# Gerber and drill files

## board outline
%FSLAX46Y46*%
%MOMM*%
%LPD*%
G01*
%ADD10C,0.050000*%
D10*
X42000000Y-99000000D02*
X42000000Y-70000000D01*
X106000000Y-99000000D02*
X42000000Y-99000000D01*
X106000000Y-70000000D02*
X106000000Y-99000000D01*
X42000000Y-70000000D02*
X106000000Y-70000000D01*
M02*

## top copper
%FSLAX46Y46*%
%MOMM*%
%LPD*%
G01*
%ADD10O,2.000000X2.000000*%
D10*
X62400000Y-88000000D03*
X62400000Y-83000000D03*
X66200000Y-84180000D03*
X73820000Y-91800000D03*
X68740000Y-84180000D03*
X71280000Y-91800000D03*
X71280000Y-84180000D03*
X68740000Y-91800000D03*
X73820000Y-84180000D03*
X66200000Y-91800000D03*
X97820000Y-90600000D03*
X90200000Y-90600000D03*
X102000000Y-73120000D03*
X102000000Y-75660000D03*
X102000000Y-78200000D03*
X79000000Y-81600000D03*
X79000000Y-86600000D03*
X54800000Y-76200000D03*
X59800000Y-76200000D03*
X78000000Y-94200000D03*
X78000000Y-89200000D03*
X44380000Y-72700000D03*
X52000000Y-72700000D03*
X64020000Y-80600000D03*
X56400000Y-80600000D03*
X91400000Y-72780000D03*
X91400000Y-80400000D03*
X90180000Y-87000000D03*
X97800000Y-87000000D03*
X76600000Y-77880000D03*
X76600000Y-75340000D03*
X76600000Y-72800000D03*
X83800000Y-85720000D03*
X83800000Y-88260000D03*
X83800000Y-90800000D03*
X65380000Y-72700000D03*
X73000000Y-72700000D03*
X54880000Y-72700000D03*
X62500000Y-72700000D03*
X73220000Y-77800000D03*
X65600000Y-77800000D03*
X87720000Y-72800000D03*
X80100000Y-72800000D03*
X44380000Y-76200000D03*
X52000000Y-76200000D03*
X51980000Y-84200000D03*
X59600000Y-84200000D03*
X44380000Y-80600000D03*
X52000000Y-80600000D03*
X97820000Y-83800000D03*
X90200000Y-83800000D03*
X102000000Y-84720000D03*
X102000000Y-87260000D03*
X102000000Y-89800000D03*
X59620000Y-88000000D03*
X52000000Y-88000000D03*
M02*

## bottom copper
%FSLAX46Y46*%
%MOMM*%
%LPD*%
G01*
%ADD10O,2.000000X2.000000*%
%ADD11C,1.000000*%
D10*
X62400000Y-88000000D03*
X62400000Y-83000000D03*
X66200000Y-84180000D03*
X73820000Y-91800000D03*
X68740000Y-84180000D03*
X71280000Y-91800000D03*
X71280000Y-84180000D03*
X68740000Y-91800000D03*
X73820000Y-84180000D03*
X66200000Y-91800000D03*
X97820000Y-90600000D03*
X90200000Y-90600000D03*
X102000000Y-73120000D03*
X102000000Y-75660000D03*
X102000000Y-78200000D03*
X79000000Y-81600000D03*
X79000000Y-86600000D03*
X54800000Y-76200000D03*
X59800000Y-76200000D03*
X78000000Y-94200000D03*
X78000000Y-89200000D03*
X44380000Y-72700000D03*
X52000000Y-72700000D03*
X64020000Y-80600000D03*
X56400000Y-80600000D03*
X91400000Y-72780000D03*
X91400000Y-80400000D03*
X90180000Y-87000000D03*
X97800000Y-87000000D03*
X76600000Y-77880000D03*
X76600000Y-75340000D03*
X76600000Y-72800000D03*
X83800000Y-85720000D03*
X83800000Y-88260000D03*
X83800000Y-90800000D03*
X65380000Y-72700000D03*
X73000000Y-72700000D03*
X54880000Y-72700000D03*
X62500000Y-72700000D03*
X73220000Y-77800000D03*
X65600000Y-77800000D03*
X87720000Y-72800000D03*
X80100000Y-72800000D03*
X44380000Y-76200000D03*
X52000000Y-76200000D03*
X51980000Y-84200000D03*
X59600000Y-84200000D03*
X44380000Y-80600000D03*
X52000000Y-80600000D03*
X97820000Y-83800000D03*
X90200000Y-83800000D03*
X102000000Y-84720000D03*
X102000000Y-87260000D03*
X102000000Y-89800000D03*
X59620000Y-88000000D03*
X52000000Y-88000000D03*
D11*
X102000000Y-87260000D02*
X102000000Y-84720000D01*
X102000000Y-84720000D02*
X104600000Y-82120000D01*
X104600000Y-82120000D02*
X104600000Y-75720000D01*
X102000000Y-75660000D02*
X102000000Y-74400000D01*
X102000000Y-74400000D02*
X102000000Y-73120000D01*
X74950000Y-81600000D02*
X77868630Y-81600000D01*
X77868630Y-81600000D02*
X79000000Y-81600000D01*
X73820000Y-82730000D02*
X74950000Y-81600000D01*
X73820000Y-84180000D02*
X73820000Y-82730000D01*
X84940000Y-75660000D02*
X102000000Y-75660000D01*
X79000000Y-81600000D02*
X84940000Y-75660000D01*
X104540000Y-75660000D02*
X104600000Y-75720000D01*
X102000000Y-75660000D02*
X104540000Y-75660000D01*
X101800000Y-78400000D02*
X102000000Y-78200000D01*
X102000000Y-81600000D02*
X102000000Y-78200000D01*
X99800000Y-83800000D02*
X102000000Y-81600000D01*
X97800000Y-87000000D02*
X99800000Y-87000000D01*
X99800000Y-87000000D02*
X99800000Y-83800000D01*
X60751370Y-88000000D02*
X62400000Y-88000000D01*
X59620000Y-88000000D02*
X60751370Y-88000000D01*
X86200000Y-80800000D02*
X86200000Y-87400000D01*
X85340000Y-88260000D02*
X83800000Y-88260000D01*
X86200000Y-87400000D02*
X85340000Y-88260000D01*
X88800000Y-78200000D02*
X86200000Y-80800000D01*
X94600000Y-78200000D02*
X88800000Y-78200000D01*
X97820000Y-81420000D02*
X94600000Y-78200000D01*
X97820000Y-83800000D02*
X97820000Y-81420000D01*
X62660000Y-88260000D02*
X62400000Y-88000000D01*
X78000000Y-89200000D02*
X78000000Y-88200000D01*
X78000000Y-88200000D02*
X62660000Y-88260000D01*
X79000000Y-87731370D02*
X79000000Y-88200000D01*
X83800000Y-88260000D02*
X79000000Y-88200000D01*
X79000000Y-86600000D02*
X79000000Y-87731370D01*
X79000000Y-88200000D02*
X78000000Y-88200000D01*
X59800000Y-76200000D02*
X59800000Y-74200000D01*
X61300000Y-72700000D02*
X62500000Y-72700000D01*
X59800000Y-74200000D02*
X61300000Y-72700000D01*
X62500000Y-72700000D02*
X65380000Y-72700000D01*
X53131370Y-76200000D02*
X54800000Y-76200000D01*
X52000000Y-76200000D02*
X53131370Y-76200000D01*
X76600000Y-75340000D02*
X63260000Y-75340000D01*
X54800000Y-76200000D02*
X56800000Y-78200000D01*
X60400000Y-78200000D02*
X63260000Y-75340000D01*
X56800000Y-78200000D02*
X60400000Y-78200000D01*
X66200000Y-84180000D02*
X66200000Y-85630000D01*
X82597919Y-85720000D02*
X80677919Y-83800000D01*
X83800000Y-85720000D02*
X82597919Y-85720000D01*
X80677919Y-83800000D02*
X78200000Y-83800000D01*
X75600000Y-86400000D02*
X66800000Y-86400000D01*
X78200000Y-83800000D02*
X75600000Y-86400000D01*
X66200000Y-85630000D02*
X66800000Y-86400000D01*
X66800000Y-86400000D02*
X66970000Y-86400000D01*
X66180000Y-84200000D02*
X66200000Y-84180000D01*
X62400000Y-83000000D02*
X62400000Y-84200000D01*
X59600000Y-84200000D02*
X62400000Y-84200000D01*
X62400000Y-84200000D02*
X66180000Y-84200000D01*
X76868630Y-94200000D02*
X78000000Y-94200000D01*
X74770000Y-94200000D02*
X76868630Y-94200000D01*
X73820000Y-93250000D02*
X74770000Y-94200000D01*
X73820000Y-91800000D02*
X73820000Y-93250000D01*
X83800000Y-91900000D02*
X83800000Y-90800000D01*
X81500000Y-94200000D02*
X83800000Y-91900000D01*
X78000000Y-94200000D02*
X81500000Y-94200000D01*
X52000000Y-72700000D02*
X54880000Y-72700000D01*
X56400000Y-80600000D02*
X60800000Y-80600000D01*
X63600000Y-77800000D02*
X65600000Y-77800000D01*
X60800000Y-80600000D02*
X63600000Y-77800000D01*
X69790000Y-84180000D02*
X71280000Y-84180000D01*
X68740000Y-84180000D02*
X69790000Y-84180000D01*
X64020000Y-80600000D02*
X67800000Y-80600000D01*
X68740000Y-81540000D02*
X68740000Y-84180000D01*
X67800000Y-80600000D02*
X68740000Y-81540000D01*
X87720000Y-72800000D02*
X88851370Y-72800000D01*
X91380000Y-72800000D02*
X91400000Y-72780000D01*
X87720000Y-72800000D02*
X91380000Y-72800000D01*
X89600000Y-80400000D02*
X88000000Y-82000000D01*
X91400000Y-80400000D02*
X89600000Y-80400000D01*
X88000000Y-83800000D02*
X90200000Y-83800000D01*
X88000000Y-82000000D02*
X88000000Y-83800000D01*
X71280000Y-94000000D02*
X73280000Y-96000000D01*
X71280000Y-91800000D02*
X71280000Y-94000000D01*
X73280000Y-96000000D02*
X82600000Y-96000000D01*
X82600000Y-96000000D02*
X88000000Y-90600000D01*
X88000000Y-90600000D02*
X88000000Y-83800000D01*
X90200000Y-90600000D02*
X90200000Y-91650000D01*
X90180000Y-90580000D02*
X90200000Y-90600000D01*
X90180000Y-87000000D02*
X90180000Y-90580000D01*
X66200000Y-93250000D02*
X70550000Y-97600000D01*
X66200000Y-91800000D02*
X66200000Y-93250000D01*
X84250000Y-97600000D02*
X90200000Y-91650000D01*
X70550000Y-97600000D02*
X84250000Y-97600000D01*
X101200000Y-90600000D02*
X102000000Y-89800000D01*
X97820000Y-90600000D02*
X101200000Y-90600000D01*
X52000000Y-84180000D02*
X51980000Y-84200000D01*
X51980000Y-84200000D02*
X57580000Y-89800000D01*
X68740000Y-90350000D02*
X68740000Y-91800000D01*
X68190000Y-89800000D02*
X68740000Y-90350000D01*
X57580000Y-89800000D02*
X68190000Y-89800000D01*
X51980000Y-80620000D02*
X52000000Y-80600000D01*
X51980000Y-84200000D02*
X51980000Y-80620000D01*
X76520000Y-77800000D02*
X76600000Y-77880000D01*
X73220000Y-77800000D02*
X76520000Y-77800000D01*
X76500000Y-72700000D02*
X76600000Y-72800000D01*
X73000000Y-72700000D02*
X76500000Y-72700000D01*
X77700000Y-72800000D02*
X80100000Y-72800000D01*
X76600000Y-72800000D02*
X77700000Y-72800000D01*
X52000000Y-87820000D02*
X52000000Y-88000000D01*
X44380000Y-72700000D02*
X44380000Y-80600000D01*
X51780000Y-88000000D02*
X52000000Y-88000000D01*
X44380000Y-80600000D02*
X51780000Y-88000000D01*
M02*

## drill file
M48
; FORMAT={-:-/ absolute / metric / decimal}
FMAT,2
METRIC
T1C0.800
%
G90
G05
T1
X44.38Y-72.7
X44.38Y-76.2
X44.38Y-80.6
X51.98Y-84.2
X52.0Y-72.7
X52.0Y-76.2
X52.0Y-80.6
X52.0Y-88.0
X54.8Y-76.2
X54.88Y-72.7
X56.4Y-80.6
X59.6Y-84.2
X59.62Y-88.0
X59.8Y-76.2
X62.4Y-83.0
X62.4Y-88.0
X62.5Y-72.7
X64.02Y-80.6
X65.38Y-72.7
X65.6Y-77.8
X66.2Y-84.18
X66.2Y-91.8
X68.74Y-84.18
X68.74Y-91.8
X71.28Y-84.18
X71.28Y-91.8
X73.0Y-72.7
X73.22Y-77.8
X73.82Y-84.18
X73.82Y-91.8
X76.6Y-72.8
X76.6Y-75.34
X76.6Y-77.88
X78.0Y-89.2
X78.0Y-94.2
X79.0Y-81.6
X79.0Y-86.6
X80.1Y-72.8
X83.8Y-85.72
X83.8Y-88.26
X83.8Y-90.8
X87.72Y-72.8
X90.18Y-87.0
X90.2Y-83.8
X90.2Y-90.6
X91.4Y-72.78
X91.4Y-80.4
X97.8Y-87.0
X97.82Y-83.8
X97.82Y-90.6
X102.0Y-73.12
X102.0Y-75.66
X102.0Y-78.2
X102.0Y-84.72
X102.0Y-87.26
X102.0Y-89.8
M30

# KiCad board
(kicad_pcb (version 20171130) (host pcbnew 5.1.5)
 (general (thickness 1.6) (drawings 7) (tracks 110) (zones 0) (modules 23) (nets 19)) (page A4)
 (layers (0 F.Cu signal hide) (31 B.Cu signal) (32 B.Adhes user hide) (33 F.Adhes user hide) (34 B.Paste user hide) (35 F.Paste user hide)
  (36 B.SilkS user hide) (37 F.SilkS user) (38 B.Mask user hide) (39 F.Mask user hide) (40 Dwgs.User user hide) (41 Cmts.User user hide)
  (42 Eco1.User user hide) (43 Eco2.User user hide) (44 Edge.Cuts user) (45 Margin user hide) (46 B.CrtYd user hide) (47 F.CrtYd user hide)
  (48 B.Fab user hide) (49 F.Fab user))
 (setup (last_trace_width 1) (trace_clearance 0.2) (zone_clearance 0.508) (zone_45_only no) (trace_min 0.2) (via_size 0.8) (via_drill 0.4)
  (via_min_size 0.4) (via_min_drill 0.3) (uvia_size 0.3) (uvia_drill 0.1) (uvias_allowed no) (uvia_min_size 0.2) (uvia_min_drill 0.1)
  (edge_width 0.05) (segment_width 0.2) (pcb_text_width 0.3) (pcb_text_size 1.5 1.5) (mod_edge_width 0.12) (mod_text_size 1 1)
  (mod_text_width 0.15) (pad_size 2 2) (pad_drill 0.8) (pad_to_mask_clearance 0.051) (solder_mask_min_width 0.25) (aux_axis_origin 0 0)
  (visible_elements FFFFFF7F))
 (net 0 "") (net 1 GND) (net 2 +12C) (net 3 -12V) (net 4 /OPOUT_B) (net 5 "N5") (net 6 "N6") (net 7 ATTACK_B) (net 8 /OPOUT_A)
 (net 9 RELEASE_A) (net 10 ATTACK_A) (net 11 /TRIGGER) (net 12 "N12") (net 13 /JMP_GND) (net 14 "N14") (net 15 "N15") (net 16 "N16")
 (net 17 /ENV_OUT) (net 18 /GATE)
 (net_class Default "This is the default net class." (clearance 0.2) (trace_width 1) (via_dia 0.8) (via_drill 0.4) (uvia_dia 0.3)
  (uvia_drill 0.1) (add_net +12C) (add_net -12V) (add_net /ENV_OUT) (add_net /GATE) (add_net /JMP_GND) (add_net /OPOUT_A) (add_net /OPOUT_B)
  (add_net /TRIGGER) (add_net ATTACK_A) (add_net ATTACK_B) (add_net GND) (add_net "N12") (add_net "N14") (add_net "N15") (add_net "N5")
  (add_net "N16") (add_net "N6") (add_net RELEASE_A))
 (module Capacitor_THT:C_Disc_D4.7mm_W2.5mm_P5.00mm (layer F.Cu) (at 62.4 83 270)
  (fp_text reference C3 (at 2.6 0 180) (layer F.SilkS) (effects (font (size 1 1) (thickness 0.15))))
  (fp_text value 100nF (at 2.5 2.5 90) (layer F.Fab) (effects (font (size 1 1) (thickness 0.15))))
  (pad 2 thru_hole oval (at 5 0 270) (size 2 2) (drill 0.8) (layers *.Cu *.Mask) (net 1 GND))
  (pad 1 thru_hole oval (at 0 0 270) (size 2 2) (drill 0.8) (layers *.Cu *.Mask) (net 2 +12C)))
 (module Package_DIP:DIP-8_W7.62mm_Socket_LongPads (layer F.Cu) (at 66.2 91.8 90)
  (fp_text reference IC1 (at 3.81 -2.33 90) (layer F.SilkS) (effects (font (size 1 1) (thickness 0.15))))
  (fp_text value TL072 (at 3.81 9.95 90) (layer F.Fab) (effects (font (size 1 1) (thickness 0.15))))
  (pad 8 thru_hole oval (at 7.62 0 90) (size 2 2) (drill 0.8) (layers *.Cu *.Mask) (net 2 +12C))
  (pad 4 thru_hole oval (at 0 7.62 90) (size 2 2) (drill 0.8) (layers *.Cu *.Mask) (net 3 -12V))
  (pad 7 thru_hole oval (at 7.62 2.54 90) (size 2 2) (drill 0.8) (layers *.Cu *.Mask) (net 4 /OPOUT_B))
  (pad 3 thru_hole oval (at 0 5.08 90) (size 2 2) (drill 0.8) (layers *.Cu *.Mask) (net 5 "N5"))
  (pad 6 thru_hole oval (at 7.62 5.08 90) (size 2 2) (drill 0.8) (layers *.Cu *.Mask) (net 4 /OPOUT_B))
  (pad 2 thru_hole oval (at 0 2.54 90) (size 2 2) (drill 0.8) (layers *.Cu *.Mask) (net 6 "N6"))
  (pad 5 thru_hole oval (at 7.62 7.62 90) (size 2 2) (drill 0.8) (layers *.Cu *.Mask) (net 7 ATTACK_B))
  (pad 1 thru_hole oval (at 0 0 90) (size 2 2) (drill 0.8) (layers *.Cu *.Mask) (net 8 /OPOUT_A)))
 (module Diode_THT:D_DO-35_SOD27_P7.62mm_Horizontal (layer F.Cu) (at 90.2 90.6)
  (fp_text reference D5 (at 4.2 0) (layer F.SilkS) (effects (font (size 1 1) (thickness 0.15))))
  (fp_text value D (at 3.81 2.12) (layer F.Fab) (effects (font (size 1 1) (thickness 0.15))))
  (pad 2 thru_hole oval (at 7.62 0) (size 2 2) (drill 0.8) (layers *.Cu *.Mask) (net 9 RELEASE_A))
  (pad 1 thru_hole oval (at 0 0) (size 2 2) (drill 0.8) (layers *.Cu *.Mask) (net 8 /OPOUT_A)))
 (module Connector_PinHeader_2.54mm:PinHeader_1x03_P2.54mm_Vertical (layer F.Cu) (at 102 78.2 180)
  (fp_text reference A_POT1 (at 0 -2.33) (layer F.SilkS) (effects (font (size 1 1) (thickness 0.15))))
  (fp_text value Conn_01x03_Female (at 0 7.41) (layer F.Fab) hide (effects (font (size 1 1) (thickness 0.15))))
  (pad 3 thru_hole oval (at 0 5.08 180) (size 2 2) (drill 0.8) (layers *.Cu *.Mask) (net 7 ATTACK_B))
  (pad 2 thru_hole oval (at 0 2.54 180) (size 2 2) (drill 0.8) (layers *.Cu *.Mask) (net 7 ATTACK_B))
  (pad 1 thru_hole oval (at 0 0 180) (size 2 2) (drill 0.8) (layers *.Cu *.Mask) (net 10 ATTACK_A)))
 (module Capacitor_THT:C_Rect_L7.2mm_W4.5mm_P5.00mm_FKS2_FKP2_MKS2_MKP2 (layer F.Cu) (at 79 86.6 90)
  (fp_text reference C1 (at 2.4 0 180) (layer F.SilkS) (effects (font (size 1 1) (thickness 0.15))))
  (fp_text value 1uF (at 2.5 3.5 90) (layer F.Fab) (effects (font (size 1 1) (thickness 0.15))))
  (pad 2 thru_hole oval (at 5 0 90) (size 2 2) (drill 0.8) (layers *.Cu *.Mask) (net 7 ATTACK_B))
  (pad 1 thru_hole oval (at 0 0 90) (size 2 2) (drill 0.8) (layers *.Cu *.Mask) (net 1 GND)))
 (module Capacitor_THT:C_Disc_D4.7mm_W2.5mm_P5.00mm (layer F.Cu) (at 59.8 76.2 180)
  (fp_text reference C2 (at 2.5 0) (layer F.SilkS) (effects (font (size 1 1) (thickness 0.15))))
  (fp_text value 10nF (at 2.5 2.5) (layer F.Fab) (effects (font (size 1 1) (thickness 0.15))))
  (pad 2 thru_hole oval (at 5 0 180) (size 2 2) (drill 0.8) (layers *.Cu *.Mask) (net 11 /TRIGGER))
  (pad 1 thru_hole oval (at 0 0 180) (size 2 2) (drill 0.8) (layers *.Cu *.Mask) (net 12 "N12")))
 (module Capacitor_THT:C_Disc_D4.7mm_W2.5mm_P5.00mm (layer F.Cu) (at 78 89.2 270)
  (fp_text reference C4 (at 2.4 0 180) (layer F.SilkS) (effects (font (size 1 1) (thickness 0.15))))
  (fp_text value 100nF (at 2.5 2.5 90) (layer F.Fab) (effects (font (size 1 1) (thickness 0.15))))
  (pad 2 thru_hole oval (at 5 0 270) (size 2 2) (drill 0.8) (layers *.Cu *.Mask) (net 3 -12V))
  (pad 1 thru_hole oval (at 0 0 270) (size 2 2) (drill 0.8) (layers *.Cu *.Mask) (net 1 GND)))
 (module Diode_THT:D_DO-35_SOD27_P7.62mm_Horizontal (layer F.Cu) (at 52 72.7 180)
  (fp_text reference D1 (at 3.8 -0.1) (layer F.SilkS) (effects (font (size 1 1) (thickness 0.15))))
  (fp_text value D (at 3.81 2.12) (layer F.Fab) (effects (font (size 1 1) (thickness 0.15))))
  (pad 2 thru_hole oval (at 7.62 0 180) (size 2 2) (drill 0.8) (layers *.Cu *.Mask) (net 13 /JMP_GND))
  (pad 1 thru_hole oval (at 0 0 180) (size 2 2) (drill 0.8) (layers *.Cu *.Mask) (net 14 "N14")))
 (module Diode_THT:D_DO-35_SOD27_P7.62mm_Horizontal (layer F.Cu) (at 56.4 80.6)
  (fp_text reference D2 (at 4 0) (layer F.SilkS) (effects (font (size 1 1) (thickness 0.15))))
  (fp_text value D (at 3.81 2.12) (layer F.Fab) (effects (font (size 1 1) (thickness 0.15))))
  (pad 2 thru_hole oval (at 7.62 0) (size 2 2) (drill 0.8) (layers *.Cu *.Mask) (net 4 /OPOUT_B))
  (pad 1 thru_hole oval (at 0 0) (size 2 2) (drill 0.8) (layers *.Cu *.Mask) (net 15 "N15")))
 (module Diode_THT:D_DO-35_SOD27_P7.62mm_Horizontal (layer F.Cu) (at 91.4 80.4 90)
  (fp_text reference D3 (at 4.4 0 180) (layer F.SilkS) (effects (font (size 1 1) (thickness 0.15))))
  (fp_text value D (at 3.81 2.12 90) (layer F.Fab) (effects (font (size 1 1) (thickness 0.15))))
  (pad 2 thru_hole oval (at 7.62 0 90) (size 2 2) (drill 0.8) (layers *.Cu *.Mask) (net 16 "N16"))
  (pad 1 thru_hole oval (at 0 0 90) (size 2 2) (drill 0.8) (layers *.Cu *.Mask) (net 5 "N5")))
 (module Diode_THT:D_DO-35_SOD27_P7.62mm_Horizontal (layer F.Cu) (at 97.8 87 180)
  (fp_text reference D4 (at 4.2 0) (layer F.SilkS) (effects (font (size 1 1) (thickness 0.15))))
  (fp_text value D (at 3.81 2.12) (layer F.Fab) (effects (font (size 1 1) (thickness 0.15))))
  (pad 2 thru_hole oval (at 7.62 0 180) (size 2 2) (drill 0.8) (layers *.Cu *.Mask) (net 8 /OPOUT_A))
  (pad 1 thru_hole oval (at 0 0 180) (size 2 2) (drill 0.8) (layers *.Cu *.Mask) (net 10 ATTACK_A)))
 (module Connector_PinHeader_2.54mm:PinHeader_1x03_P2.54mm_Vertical (layer F.Cu) (at 76.6 72.8)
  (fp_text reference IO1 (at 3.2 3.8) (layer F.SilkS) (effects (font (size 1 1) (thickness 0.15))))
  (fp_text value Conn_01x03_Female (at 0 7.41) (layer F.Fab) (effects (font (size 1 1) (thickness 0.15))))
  (pad 3 thru_hole oval (at 0 5.08) (size 2 2) (drill 0.8) (layers *.Cu *.Mask) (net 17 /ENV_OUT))
  (pad 2 thru_hole oval (at 0 2.54) (size 2 2) (drill 0.8) (layers *.Cu *.Mask) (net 11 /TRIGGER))
  (pad 1 thru_hole oval (at 0 0) (size 2 2) (drill 0.8) (layers *.Cu *.Mask) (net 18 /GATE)))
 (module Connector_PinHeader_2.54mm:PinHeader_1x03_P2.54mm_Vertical (layer F.Cu) (at 83.8 90.8 180)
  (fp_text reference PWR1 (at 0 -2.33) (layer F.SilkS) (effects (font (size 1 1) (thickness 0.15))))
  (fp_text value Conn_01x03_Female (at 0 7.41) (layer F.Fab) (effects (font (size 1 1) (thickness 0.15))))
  (pad 3 thru_hole oval (at 0 5.08 180) (size 2 2) (drill 0.8) (layers *.Cu *.Mask) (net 2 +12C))
  (pad 2 thru_hole oval (at 0 2.54 180) (size 2 2) (drill 0.8) (layers *.Cu *.Mask) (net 1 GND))
  (pad 1 thru_hole oval (at 0 0 180) (size 2 2) (drill 0.8) (layers *.Cu *.Mask) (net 3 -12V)))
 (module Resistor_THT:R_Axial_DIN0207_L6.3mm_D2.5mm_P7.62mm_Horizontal (layer F.Cu) (at 73 72.7 180)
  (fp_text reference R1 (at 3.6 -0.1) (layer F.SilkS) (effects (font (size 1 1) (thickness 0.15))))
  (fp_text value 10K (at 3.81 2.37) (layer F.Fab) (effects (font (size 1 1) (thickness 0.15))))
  (pad 2 thru_hole oval (at 7.62 0 180) (size 2 2) (drill 0.8) (layers *.Cu *.Mask) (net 12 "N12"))
  (pad 1 thru_hole oval (at 0 0 180) (size 2 2) (drill 0.8) (layers *.Cu *.Mask) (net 18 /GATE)))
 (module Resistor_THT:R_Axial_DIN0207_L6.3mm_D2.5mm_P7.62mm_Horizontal (layer F.Cu) (at 62.5 72.7 180)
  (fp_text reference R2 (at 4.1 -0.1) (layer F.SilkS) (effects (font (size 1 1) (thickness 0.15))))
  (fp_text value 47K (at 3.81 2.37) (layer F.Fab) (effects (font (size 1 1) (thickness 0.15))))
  (pad 2 thru_hole oval (at 7.62 0 180) (size 2 2) (drill 0.8) (layers *.Cu *.Mask) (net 14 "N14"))
  (pad 1 thru_hole oval (at 0 0 180) (size 2 2) (drill 0.8) (layers *.Cu *.Mask) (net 12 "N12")))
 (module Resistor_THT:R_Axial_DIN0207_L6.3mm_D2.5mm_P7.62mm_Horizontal (layer F.Cu) (at 65.6 77.8)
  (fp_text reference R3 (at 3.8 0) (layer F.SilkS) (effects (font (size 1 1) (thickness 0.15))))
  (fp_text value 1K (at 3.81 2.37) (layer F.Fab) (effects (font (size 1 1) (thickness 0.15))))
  (pad 2 thru_hole oval (at 7.62 0) (size 2 2) (drill 0.8) (layers *.Cu *.Mask) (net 17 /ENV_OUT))
  (pad 1 thru_hole oval (at 0 0) (size 2 2) (drill 0.8) (layers *.Cu *.Mask) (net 15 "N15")))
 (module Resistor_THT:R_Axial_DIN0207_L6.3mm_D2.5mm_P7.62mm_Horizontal (layer F.Cu) (at 80.1 72.8)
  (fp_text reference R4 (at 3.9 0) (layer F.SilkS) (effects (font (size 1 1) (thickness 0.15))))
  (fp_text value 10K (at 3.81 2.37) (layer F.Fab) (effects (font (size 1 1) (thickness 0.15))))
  (pad 2 thru_hole oval (at 7.62 0) (size 2 2) (drill 0.8) (layers *.Cu *.Mask) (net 16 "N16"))
  (pad 1 thru_hole oval (at 0 0) (size 2 2) (drill 0.8) (layers *.Cu *.Mask) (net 18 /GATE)))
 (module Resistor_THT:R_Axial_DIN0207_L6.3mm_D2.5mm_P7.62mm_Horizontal (layer F.Cu) (at 52 76.2 180)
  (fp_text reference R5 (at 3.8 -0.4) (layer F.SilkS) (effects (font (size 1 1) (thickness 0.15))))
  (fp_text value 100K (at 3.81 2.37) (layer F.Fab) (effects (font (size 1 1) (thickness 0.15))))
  (pad 2 thru_hole oval (at 7.62 0 180) (size 2 2) (drill 0.8) (layers *.Cu *.Mask) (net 13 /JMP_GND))
  (pad 1 thru_hole oval (at 0 0 180) (size 2 2) (drill 0.8) (layers *.Cu *.Mask) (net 11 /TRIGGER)))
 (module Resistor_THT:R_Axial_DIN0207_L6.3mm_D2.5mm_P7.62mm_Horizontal (layer F.Cu) (at 59.6 84.2 180)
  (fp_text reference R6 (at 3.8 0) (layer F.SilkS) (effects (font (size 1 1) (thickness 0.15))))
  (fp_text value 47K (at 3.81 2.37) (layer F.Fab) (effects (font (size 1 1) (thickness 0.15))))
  (pad 2 thru_hole oval (at 7.62 0 180) (size 2 2) (drill 0.8) (layers *.Cu *.Mask) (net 6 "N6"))
  (pad 1 thru_hole oval (at 0 0 180) (size 2 2) (drill 0.8) (layers *.Cu *.Mask) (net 2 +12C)))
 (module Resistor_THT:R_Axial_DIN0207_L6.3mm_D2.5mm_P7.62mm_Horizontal (layer F.Cu) (at 52 80.6 180)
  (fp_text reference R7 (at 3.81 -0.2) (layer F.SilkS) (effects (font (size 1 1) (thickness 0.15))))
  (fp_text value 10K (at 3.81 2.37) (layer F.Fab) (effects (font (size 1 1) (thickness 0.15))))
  (pad 2 thru_hole oval (at 7.62 0 180) (size 2 2) (drill 0.8) (layers *.Cu *.Mask) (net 13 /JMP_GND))
  (pad 1 thru_hole oval (at 0 0 180) (size 2 2) (drill 0.8) (layers *.Cu *.Mask) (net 6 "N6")))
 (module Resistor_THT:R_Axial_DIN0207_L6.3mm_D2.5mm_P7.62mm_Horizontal (layer F.Cu) (at 90.2 83.8)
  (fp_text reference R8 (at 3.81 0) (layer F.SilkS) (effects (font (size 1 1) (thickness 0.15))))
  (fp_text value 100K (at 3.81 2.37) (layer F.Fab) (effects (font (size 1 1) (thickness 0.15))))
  (pad 2 thru_hole oval (at 7.62 0) (size 2 2) (drill 0.8) (layers *.Cu *.Mask) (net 1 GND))
  (pad 1 thru_hole oval (at 0 0) (size 2 2) (drill 0.8) (layers *.Cu *.Mask) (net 5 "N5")))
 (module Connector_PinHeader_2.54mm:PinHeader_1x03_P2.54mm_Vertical (layer F.Cu) (at 102 89.8 180)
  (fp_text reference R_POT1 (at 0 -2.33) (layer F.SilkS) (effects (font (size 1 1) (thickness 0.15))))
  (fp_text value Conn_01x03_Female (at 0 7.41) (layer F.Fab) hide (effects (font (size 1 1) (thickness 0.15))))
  (pad 3 thru_hole oval (at 0 5.08 180) (size 2 2) (drill 0.8) (layers *.Cu *.Mask) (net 7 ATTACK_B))
  (pad 2 thru_hole oval (at 0 2.54 180) (size 2 2) (drill 0.8) (layers *.Cu *.Mask) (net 7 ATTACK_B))
  (pad 1 thru_hole oval (at 0 0 180) (size 2 2) (drill 0.8) (layers *.Cu *.Mask) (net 9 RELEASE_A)))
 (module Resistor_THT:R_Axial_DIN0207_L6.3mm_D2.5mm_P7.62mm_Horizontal (layer F.Cu) (at 52 88)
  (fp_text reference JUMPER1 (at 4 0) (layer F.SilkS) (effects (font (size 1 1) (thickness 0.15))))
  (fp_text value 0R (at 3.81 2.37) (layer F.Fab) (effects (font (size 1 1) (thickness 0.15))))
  (pad 2 thru_hole oval (at 7.62 0) (size 2 2) (drill 0.8) (layers *.Cu *.Mask) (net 1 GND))
  (pad 1 thru_hole oval (at 0 0) (size 2 2) (drill 0.8) (layers *.Cu *.Mask) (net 13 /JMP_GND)))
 (gr_line (start 42 99) (end 42 70) (layer Edge.Cuts) (width 0.05))
 (gr_line (start 106 99) (end 42 99) (layer Edge.Cuts) (width 0.05))
 (gr_line (start 106 70) (end 106 99) (layer Edge.Cuts) (width 0.05))
 (gr_line (start 42 70) (end 106 70) (layer Edge.Cuts) (width 0.05))
 (segment (start 102 87.26) (end 102 84.72) (width 1) (layer B.Cu) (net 7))
 (segment (start 102 84.72) (end 104.6 82.12) (width 1) (layer B.Cu) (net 7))
 (segment (start 104.6 82.12) (end 104.6 75.72) (width 1) (layer B.Cu) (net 7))
 (segment (start 102 75.66) (end 102 74.4) (width 1) (layer B.Cu) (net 7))
 (segment (start 102 74.4) (end 102 73.12) (width 1) (layer B.Cu) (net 7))
 (segment (start 74.95 81.6) (end 77.86863 81.6) (width 1) (layer B.Cu) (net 7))
 (segment (start 77.86863 81.6) (end 79 81.6) (width 1) (layer B.Cu) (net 7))
 (segment (start 73.82 82.73) (end 74.95 81.6) (width 1) (layer B.Cu) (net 7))
 (segment (start 73.82 84.18) (end 73.82 82.73) (width 1) (layer B.Cu) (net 7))
 (segment (start 84.94 75.66) (end 102 75.66) (width 1) (layer B.Cu) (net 7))
 (segment (start 79 81.6) (end 84.94 75.66) (width 1) (layer B.Cu) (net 7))
 (segment (start 104.54 75.66) (end 104.6 75.72) (width 1) (layer B.Cu) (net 7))
 (segment (start 102 75.66) (end 104.54 75.66) (width 1) (layer B.Cu) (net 7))
 (segment (start 101.8 78.4) (end 102 78.2) (width 1) (layer B.Cu) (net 10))
 (segment (start 102 81.6) (end 102 78.2) (width 1) (layer B.Cu) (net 10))
 (segment (start 99.8 83.8) (end 102 81.6) (width 1) (layer B.Cu) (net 10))
 (segment (start 97.8 87) (end 99.8 87) (width 1) (layer B.Cu) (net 10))
 (segment (start 99.8 87) (end 99.8 83.8) (width 1) (layer B.Cu) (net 10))
 (segment (start 60.75137 88) (end 62.4 88) (width 1) (layer B.Cu) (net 1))
 (segment (start 59.62 88) (end 60.75137 88) (width 1) (layer B.Cu) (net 1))
 (segment (start 86.2 80.8) (end 86.2 87.4) (width 1) (layer B.Cu) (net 1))
 (segment (start 85.34 88.26) (end 83.8 88.26) (width 1) (layer B.Cu) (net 1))
 (segment (start 86.2 87.4) (end 85.34 88.26) (width 1) (layer B.Cu) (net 1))
 (segment (start 88.8 78.2) (end 86.2 80.8) (width 1) (layer B.Cu) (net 1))
 (segment (start 94.6 78.2) (end 88.8 78.2) (width 1) (layer B.Cu) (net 1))
 (segment (start 97.82 81.42) (end 94.6 78.2) (width 1) (layer B.Cu) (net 1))
 (segment (start 97.82 83.8) (end 97.82 81.42) (width 1) (layer B.Cu) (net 1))
 (segment (start 62.66 88.26) (end 62.4 88) (width 1) (layer B.Cu) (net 1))
 (segment (start 78 89.2) (end 78 88.2) (width 1) (layer B.Cu) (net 1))
 (segment (start 78 88.2) (end 62.66 88.26) (width 1) (layer B.Cu) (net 1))
 (segment (start 79 87.73137) (end 79 88.2) (width 1) (layer B.Cu) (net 1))
 (segment (start 83.8 88.26) (end 79 88.2) (width 1) (layer B.Cu) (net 1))
 (segment (start 79 86.6) (end 79 87.73137) (width 1) (layer B.Cu) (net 1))
 (segment (start 79 88.2) (end 78 88.2) (width 1) (layer B.Cu) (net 1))
 (segment (start 59.8 76.2) (end 59.8 74.2) (width 1) (layer B.Cu) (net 12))
 (segment (start 61.3 72.7) (end 62.5 72.7) (width 1) (layer B.Cu) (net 12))
 (segment (start 59.8 74.2) (end 61.3 72.7) (width 1) (layer B.Cu) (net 12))
 (segment (start 62.5 72.7) (end 65.38 72.7) (width 1) (layer B.Cu) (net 12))
 (segment (start 53.13137 76.2) (end 54.8 76.2) (width 1) (layer B.Cu) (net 11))
 (segment (start 52 76.2) (end 53.13137 76.2) (width 1) (layer B.Cu) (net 11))
 (segment (start 76.6 75.34) (end 63.26 75.34) (width 1) (layer B.Cu) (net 11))
 (segment (start 54.8 76.2) (end 56.8 78.2) (width 1) (layer B.Cu) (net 11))
 (segment (start 60.4 78.2) (end 63.26 75.34) (width 1) (layer B.Cu) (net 11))
 (segment (start 56.8 78.2) (end 60.4 78.2) (width 1) (layer B.Cu) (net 11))
 (segment (start 66.2 84.18) (end 66.2 85.63) (width 1) (layer B.Cu) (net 2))
 (segment (start 82.597919 85.72) (end 80.677919 83.8) (width 1) (layer B.Cu) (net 2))
 (segment (start 83.8 85.72) (end 82.597919 85.72) (width 1) (layer B.Cu) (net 2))
 (segment (start 80.677919 83.8) (end 78.2 83.8) (width 1) (layer B.Cu) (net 2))
 (segment (start 75.6 86.4) (end 66.8 86.4) (width 1) (layer B.Cu) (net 2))
 (segment (start 78.2 83.8) (end 75.6 86.4) (width 1) (layer B.Cu) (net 2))
 (segment (start 66.2 85.63) (end 66.8 86.4) (width 1) (layer B.Cu) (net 2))
 (segment (start 66.8 86.4) (end 66.97 86.4) (width 1) (layer B.Cu) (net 2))
 (segment (start 66.18 84.2) (end 66.2 84.18) (width 1) (layer B.Cu) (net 2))
 (segment (start 62.4 83) (end 62.4 84.2) (width 1) (layer B.Cu) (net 2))
 (segment (start 59.6 84.2) (end 62.4 84.2) (width 1) (layer B.Cu) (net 2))
 (segment (start 62.4 84.2) (end 66.18 84.2) (width 1) (layer B.Cu) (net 2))
 (segment (start 76.86863 94.2) (end 78 94.2) (width 1) (layer B.Cu) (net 3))
 (segment (start 74.77 94.2) (end 76.86863 94.2) (width 1) (layer B.Cu) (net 3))
 (segment (start 73.82 93.25) (end 74.77 94.2) (width 1) (layer B.Cu) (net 3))
 (segment (start 73.82 91.8) (end 73.82 93.25) (width 1) (layer B.Cu) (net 3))
 (segment (start 83.8 91.9) (end 83.8 90.8) (width 1) (layer B.Cu) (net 3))
 (segment (start 81.5 94.2) (end 83.8 91.9) (width 1) (layer B.Cu) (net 3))
 (segment (start 78 94.2) (end 81.5 94.2) (width 1) (layer B.Cu) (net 3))
 (segment (start 52 72.7) (end 54.88 72.7) (width 1) (layer B.Cu) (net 14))
 (segment (start 56.4 80.6) (end 60.8 80.6) (width 1) (layer B.Cu) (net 15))
 (segment (start 63.6 77.8) (end 65.6 77.8) (width 1) (layer B.Cu) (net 15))
 (segment (start 60.8 80.6) (end 63.6 77.8) (width 1) (layer B.Cu) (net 15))
 (segment (start 69.79 84.18) (end 71.28 84.18) (width 1) (layer B.Cu) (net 4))
 (segment (start 68.74 84.18) (end 69.79 84.18) (width 1) (layer B.Cu) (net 4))
 (segment (start 64.02 80.6) (end 67.8 80.6) (width 1) (layer B.Cu) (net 4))
 (segment (start 68.74 81.54) (end 68.74 84.18) (width 1) (layer B.Cu) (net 4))
 (segment (start 67.8 80.6) (end 68.74 81.54) (width 1) (layer B.Cu) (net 4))
 (segment (start 87.72 72.8) (end 88.85137 72.8) (width 1) (layer B.Cu) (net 16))
 (segment (start 91.38 72.8) (end 91.4 72.78) (width 1) (layer B.Cu) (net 16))
 (segment (start 87.72 72.8) (end 91.38 72.8) (width 1) (layer B.Cu) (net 16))
 (segment (start 89.6 80.4) (end 88 82) (width 1) (layer B.Cu) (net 5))
 (segment (start 91.4 80.4) (end 89.6 80.4) (width 1) (layer B.Cu) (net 5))
 (segment (start 88 83.8) (end 90.2 83.8) (width 1) (layer B.Cu) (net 5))
 (segment (start 88 82) (end 88 83.8) (width 1) (layer B.Cu) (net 5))
 (segment (start 71.28 94) (end 73.28 96) (width 1) (layer B.Cu) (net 5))
 (segment (start 71.28 91.8) (end 71.28 94) (width 1) (layer B.Cu) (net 5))
 (segment (start 73.28 96) (end 82.6 96) (width 1) (layer B.Cu) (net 5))
 (segment (start 82.6 96) (end 88 90.6) (width 1) (layer B.Cu) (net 5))
 (segment (start 88 90.6) (end 88 83.8) (width 1) (layer B.Cu) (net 5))
 (segment (start 90.2 90.6) (end 90.2 91.65) (width 1) (layer B.Cu) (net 8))
 (segment (start 90.18 90.58) (end 90.2 90.6) (width 1) (layer B.Cu) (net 8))
 (segment (start 90.18 87) (end 90.18 90.58) (width 1) (layer B.Cu) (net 8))
 (segment (start 66.2 93.25) (end 70.55 97.6) (width 1) (layer B.Cu) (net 8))
 (segment (start 66.2 91.8) (end 66.2 93.25) (width 1) (layer B.Cu) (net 8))
 (segment (start 84.25 97.6) (end 90.2 91.65) (width 1) (layer B.Cu) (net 8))
 (segment (start 70.55 97.6) (end 84.25 97.6) (width 1) (layer B.Cu) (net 8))
 (segment (start 101.2 90.6) (end 102 89.8) (width 1) (layer B.Cu) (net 9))
 (segment (start 97.82 90.6) (end 101.2 90.6) (width 1) (layer B.Cu) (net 9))
 (segment (start 52 84.18) (end 51.98 84.2) (width 1) (layer B.Cu) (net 6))
 (segment (start 51.98 84.2) (end 57.58 89.8) (width 1) (layer B.Cu) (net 6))
 (segment (start 68.74 90.35) (end 68.74 91.8) (width 1) (layer B.Cu) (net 6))
 (segment (start 68.19 89.8) (end 68.74 90.35) (width 1) (layer B.Cu) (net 6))
 (segment (start 57.58 89.8) (end 68.19 89.8) (width 1) (layer B.Cu) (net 6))
 (segment (start 51.98 80.62) (end 52 80.6) (width 1) (layer B.Cu) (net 6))
 (segment (start 51.98 84.2) (end 51.98 80.62) (width 1) (layer B.Cu) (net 6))
 (segment (start 76.52 77.8) (end 76.6 77.88) (width 1) (layer B.Cu) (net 17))
 (segment (start 73.22 77.8) (end 76.52 77.8) (width 1) (layer B.Cu) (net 17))
 (segment (start 76.5 72.7) (end 76.6 72.8) (width 1) (layer B.Cu) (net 18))
 (segment (start 73 72.7) (end 76.5 72.7) (width 1) (layer B.Cu) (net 18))
 (segment (start 77.7 72.8) (end 80.1 72.8) (width 1) (layer B.Cu) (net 18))
 (segment (start 76.6 72.8) (end 77.7 72.8) (width 1) (layer B.Cu) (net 18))
 (segment (start 52 87.82) (end 52 88) (width 1) (layer B.Cu) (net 13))
 (segment (start 44.38 72.7) (end 44.38 80.6) (width 1) (layer B.Cu) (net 13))
 (segment (start 51.78 88) (end 52 88) (width 1) (layer B.Cu) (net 13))
 (segment (start 44.38 80.6) (end 51.78 88) (width 1) (layer B.Cu) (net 13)))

